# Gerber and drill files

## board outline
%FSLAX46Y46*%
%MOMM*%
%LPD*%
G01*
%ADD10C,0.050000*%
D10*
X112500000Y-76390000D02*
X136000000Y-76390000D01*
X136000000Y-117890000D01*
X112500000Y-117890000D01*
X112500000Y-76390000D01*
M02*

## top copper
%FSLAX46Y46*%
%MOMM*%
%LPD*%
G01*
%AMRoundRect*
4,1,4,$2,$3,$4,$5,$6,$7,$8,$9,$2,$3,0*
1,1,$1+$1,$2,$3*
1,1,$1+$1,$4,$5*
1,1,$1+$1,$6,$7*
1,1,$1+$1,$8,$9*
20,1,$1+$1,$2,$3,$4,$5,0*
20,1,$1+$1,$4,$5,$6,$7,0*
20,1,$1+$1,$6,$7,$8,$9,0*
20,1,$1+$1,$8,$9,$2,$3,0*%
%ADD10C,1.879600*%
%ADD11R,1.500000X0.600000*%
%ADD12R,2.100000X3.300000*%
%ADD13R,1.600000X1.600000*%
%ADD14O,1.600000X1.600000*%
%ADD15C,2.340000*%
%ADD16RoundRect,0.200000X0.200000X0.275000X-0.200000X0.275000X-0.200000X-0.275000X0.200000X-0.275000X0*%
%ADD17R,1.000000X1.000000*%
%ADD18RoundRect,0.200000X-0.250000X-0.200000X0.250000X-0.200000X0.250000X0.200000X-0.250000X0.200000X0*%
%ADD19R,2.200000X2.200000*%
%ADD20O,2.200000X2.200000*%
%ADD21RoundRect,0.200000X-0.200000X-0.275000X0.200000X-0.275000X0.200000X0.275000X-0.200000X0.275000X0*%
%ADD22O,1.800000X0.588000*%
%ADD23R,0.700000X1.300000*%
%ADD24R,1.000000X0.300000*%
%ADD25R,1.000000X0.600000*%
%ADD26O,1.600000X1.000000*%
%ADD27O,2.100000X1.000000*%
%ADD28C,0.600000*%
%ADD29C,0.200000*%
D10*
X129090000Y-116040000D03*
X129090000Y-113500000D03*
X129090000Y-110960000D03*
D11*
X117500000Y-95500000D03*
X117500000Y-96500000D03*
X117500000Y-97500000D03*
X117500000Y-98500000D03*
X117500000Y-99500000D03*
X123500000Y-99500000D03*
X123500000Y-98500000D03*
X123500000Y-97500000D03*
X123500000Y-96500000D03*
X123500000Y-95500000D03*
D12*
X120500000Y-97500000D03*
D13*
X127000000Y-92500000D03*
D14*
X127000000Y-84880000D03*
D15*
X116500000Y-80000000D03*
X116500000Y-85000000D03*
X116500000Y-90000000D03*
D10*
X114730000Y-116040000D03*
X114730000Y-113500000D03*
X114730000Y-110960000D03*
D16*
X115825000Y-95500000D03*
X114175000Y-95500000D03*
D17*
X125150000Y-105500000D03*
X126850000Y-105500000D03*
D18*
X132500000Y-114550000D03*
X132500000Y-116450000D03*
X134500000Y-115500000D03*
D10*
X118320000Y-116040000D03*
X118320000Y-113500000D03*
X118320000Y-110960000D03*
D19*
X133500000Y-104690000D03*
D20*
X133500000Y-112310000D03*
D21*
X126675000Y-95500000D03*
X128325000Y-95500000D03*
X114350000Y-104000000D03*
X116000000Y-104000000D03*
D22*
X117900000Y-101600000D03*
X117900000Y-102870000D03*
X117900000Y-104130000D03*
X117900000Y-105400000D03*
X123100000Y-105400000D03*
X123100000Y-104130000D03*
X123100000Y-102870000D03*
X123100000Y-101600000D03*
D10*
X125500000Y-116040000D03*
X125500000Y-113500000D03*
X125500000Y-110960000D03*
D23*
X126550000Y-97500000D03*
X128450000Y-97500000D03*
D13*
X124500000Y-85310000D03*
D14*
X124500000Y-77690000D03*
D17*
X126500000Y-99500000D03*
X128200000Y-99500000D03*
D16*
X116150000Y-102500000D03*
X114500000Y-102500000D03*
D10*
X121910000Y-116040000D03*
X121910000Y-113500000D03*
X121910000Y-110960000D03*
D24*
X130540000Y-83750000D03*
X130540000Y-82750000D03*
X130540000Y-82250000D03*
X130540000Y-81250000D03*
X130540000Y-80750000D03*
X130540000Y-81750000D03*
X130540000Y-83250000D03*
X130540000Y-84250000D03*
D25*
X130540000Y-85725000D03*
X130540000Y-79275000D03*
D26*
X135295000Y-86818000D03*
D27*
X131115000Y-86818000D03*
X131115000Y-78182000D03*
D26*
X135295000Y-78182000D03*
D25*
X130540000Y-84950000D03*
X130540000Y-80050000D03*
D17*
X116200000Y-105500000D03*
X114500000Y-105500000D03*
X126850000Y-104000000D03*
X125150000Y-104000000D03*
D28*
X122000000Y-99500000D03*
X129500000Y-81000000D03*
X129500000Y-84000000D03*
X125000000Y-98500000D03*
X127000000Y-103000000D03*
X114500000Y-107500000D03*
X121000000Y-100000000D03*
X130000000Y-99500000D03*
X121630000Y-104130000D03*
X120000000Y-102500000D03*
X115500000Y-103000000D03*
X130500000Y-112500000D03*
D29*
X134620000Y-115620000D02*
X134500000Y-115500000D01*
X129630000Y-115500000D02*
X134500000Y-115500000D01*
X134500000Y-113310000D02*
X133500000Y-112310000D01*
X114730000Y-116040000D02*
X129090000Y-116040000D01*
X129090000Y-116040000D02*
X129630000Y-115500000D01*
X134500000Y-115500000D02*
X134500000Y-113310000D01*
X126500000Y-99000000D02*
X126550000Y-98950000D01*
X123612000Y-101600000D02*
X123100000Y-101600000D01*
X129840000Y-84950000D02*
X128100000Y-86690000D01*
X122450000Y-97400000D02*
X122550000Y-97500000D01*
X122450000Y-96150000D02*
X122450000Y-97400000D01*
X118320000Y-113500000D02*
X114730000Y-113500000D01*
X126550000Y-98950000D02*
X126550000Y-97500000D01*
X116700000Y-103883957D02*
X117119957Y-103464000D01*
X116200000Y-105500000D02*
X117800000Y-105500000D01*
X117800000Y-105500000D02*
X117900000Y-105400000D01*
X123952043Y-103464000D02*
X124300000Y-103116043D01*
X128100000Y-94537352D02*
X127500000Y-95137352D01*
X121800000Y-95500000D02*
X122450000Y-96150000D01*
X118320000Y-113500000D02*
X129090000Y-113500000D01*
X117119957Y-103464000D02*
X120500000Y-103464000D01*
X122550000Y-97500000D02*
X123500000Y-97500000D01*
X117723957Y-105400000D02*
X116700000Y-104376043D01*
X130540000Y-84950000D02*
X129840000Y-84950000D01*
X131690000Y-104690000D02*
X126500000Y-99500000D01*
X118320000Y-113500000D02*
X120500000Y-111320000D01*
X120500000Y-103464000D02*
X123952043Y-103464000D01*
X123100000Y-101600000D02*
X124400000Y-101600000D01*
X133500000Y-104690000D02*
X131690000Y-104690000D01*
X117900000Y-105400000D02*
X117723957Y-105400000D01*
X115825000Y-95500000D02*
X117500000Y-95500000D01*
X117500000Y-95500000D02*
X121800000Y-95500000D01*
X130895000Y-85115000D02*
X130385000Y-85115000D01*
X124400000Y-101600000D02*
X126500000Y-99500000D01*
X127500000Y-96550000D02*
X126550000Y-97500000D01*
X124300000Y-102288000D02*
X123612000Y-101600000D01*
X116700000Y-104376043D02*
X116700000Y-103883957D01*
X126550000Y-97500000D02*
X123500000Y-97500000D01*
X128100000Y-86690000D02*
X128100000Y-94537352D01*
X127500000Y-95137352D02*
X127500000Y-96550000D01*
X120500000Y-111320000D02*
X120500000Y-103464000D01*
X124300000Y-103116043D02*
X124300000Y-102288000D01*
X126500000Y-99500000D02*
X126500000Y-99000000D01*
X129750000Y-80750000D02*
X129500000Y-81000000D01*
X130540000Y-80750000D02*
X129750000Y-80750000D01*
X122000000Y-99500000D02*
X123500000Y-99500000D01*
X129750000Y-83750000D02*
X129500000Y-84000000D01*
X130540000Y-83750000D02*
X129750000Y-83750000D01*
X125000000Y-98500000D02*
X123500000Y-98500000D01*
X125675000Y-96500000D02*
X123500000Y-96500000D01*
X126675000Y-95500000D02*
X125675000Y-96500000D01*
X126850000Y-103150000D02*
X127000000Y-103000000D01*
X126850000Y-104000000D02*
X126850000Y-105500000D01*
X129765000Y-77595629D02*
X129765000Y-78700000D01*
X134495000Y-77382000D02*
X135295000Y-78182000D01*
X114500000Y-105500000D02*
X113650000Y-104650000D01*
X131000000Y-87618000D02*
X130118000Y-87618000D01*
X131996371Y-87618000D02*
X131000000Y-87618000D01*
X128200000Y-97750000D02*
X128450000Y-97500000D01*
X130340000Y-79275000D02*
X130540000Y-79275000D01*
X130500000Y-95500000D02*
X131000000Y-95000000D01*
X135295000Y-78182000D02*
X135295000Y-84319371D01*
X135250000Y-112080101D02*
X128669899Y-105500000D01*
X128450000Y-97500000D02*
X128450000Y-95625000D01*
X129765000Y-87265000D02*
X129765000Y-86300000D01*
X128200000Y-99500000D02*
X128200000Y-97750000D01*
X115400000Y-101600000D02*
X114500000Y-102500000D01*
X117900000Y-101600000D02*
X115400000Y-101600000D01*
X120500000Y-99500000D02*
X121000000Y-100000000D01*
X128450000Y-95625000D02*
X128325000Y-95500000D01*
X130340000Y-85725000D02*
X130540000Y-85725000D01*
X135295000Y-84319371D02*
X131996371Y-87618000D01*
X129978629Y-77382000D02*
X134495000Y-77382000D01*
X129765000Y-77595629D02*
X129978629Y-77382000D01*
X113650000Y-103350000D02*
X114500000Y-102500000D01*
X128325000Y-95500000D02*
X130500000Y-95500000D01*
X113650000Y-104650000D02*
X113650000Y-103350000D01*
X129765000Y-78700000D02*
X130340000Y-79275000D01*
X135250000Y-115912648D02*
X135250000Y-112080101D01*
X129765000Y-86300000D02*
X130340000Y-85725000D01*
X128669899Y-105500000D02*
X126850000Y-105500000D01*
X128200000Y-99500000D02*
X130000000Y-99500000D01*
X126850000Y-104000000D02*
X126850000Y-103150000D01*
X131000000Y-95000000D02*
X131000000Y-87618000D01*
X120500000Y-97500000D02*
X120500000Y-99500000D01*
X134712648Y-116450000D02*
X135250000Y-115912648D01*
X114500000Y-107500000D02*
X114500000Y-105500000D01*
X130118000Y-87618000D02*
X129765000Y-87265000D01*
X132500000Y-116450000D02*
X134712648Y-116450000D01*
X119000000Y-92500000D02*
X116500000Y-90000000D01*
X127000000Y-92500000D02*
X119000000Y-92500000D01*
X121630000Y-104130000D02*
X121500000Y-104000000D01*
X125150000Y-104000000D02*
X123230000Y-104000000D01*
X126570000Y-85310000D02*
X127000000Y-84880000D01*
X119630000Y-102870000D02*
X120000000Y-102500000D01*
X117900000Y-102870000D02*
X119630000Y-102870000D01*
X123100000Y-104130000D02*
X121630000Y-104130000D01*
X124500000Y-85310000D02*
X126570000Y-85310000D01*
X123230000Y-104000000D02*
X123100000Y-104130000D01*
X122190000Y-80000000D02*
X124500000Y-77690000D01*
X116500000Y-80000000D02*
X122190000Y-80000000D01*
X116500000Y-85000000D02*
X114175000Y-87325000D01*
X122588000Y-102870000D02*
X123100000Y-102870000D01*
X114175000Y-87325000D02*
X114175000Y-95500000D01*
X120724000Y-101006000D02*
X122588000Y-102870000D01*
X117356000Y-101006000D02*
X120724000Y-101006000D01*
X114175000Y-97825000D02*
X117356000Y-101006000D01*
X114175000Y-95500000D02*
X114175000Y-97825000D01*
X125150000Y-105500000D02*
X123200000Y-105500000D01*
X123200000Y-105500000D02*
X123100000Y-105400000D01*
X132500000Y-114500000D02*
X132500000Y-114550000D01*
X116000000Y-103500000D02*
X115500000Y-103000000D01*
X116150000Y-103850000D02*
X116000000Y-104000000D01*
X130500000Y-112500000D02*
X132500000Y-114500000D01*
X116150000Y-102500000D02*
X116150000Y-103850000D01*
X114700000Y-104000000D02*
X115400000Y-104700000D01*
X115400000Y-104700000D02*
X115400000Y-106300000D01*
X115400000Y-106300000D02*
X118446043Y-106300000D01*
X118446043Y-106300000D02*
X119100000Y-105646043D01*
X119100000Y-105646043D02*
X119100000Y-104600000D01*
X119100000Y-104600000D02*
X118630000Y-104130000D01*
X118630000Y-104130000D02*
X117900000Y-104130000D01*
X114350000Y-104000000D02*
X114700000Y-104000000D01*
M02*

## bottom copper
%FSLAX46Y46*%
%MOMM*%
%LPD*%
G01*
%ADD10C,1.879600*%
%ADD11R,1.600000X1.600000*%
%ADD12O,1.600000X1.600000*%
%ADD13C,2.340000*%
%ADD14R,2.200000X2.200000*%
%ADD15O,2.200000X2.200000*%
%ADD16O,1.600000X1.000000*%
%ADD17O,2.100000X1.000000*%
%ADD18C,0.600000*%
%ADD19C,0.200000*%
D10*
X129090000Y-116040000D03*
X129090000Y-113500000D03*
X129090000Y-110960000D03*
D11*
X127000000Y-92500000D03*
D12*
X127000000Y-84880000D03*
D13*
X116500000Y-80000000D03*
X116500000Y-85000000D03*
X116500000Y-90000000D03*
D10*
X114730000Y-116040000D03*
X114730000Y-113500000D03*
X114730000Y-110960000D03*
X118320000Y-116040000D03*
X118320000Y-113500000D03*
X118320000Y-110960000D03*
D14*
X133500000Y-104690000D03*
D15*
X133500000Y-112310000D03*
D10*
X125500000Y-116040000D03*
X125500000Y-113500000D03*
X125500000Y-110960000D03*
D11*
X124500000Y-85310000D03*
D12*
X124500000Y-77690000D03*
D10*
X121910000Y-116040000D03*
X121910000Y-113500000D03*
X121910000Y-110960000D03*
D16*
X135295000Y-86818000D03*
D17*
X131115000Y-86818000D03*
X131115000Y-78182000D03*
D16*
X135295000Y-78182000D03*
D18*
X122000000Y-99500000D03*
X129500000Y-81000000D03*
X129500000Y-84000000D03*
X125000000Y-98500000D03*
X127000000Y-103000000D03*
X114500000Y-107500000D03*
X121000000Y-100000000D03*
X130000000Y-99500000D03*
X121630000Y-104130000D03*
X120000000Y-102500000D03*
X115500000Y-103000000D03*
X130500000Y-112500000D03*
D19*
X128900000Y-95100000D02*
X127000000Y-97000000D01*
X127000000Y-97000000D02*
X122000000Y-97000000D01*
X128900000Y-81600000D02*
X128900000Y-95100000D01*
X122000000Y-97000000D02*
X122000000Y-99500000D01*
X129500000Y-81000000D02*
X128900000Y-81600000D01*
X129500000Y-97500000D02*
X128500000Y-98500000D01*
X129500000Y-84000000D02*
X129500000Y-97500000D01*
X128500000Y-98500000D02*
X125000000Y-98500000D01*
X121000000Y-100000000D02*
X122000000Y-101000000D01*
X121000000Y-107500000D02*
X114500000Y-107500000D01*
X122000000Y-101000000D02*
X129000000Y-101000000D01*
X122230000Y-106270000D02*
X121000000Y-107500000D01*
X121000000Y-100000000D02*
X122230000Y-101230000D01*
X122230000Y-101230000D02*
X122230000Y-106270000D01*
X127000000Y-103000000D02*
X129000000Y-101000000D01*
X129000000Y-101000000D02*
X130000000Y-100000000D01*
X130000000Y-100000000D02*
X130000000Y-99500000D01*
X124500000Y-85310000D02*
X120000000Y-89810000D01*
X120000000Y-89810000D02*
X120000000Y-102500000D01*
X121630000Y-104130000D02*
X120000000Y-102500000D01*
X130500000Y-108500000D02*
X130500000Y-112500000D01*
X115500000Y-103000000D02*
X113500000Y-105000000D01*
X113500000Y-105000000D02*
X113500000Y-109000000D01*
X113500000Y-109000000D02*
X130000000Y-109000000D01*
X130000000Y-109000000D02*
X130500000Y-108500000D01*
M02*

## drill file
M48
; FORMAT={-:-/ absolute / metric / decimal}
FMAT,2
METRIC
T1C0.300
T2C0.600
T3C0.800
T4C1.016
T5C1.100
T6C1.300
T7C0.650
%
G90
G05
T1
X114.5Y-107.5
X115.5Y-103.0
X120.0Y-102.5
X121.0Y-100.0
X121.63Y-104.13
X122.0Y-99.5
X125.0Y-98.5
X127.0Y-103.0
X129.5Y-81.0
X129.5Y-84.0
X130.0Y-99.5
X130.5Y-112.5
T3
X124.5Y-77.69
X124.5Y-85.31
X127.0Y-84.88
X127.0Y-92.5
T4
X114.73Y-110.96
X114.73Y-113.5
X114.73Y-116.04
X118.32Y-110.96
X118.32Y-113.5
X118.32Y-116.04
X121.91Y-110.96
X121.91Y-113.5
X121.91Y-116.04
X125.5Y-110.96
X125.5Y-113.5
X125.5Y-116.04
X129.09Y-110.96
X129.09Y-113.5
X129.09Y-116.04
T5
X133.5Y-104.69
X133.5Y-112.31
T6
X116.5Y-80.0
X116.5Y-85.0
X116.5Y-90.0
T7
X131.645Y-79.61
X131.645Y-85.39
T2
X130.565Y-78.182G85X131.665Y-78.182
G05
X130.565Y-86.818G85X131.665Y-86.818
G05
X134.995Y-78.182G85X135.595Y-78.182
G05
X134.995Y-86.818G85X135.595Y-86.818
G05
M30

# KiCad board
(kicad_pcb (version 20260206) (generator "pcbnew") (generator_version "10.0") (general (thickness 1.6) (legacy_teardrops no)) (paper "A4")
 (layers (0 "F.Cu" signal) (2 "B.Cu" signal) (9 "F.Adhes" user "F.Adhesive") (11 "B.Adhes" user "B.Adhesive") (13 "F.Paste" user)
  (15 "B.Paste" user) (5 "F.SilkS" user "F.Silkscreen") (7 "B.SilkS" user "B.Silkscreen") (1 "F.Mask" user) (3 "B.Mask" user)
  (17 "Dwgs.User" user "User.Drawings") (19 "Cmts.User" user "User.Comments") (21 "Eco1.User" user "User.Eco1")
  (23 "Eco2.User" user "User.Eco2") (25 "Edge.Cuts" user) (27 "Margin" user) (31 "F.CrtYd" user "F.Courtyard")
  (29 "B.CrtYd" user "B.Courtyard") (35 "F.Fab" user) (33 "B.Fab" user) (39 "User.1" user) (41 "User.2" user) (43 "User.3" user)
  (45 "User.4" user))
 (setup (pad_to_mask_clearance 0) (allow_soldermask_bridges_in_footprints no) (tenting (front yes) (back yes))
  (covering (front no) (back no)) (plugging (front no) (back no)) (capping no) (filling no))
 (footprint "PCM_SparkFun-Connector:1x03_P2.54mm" (layer "F.Cu") (at 129.09 116.04 90)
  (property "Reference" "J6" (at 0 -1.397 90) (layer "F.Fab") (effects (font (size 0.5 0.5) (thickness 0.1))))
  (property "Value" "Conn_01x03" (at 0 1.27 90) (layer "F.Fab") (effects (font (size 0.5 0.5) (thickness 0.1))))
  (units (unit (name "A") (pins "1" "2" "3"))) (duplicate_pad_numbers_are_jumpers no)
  (pad "1" thru_hole circle (at 0 0 180) (size 1.8796 1.8796) (drill 1.016) (layers "*.Cu" "*.Mask") (remove_unused_layers yes)
   (keep_end_layers yes) (zone_layer_connections) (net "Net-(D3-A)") (thermal_bridge_angle 0))
  (pad "2" thru_hole circle (at 2.54 0 180) (size 1.8796 1.8796) (drill 1.016) (layers "*.Cu" "*.Mask") (remove_unused_layers yes)
   (keep_end_layers yes) (zone_layer_connections) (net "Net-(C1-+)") (thermal_bridge_angle 0))
  (pad "3" thru_hole circle (at 5.08 0 180) (size 1.8796 1.8796) (drill 1.016) (layers "*.Cu" "*.Mask") (remove_unused_layers yes)
   (keep_end_layers yes) (zone_layer_connections) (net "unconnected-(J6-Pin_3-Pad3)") (thermal_bridge_angle 0)))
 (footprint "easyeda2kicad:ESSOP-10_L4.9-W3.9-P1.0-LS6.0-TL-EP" (layer "F.Cu") (at 120.5 97.5 -90)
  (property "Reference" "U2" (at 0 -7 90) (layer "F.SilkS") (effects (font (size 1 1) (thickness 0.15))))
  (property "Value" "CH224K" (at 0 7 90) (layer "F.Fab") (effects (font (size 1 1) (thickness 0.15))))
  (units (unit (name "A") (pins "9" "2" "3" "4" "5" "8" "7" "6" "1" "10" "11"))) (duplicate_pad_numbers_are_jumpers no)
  (pad "1" smd rect (at -2 3) (size 1.5 0.6) (layers "F.Cu" "F.Mask" "F.Paste") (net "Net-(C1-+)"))
  (pad "2" smd rect (at -1 3) (size 1.5 0.6) (layers "F.Cu" "F.Mask" "F.Paste") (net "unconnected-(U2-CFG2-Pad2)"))
  (pad "3" smd rect (at 0 3) (size 1.5 0.6) (layers "F.Cu" "F.Mask" "F.Paste") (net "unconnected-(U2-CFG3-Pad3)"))
  (pad "4" smd rect (at 1 3) (size 1.5 0.6) (layers "F.Cu" "F.Mask" "F.Paste") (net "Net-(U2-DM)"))
  (pad "5" smd rect (at 2 3) (size 1.5 0.6) (layers "F.Cu" "F.Mask" "F.Paste") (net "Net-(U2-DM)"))
  (pad "6" smd rect (at 2 -3) (size 1.5 0.6) (layers "F.Cu" "F.Mask" "F.Paste") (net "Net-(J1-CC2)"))
  (pad "7" smd rect (at 1 -3) (size 1.5 0.6) (layers "F.Cu" "F.Mask" "F.Paste") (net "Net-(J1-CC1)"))
  (pad "8" smd rect (at 0 -3) (size 1.5 0.6) (layers "F.Cu" "F.Mask" "F.Paste") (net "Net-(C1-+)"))
  (pad "9" smd rect (at -1 -3) (size 1.5 0.6) (layers "F.Cu" "F.Mask" "F.Paste") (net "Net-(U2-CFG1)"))
  (pad "10" smd rect (at -2 -3) (size 1.5 0.6) (layers "F.Cu" "F.Mask" "F.Paste") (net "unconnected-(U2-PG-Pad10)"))
  (pad "11" smd rect (at 0 0 90) (size 3.3 2.1) (layers "F.Cu" "F.Mask" "F.Paste") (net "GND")))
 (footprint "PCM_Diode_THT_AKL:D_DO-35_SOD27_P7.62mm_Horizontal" (layer "F.Cu") (at 127 92.5 90)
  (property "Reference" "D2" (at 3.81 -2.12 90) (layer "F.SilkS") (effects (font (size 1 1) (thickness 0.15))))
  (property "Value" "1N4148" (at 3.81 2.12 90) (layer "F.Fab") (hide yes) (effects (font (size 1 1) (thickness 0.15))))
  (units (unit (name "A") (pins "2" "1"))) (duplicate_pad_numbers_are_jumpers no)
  (pad "1" thru_hole rect (at 0 0 90) (size 1.6 1.6) (drill 0.8) (layers "*.Cu" "*.Mask") (remove_unused_layers no) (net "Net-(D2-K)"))
  (pad "2" thru_hole oval (at 7.62 0 90) (size 1.6 1.6) (drill 0.8) (layers "*.Cu" "*.Mask") (remove_unused_layers no) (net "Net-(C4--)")))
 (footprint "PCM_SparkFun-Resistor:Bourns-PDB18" (layer "F.Cu") (at 116.5 85 180)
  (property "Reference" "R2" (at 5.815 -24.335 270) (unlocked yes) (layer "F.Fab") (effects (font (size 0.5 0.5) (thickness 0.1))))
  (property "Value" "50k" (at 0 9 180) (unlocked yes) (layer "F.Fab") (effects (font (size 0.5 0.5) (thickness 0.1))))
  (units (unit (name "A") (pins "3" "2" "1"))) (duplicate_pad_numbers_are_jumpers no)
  (pad "1" thru_hole circle (at 0 5 180) (size 2.34 2.34) (drill 1.3) (layers "*.Cu" "*.Mask") (remove_unused_layers no) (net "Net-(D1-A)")
   (thermal_bridge_angle 0))
  (pad "2" thru_hole circle (at 0 0 180) (size 2.34 2.34) (drill 1.3) (layers "*.Cu" "*.Mask") (remove_unused_layers no)
   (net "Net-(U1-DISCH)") (thermal_bridge_angle 0))
  (pad "3" thru_hole circle (at 0 -5 180) (size 2.34 2.34) (drill 1.3) (layers "*.Cu" "*.Mask") (remove_unused_layers no) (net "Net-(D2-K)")
   (thermal_bridge_angle 0)))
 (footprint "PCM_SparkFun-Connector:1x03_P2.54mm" (layer "F.Cu") (at 114.73 116.04 90)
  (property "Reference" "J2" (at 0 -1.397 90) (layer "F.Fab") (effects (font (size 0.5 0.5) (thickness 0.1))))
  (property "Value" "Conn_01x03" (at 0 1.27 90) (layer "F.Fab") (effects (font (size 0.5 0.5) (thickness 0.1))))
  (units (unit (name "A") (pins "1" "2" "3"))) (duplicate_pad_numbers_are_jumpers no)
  (pad "1" thru_hole circle (at 0 0 180) (size 1.8796 1.8796) (drill 1.016) (layers "*.Cu" "*.Mask") (remove_unused_layers yes)
   (keep_end_layers yes) (zone_layer_connections) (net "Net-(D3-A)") (thermal_bridge_angle 0))
  (pad "2" thru_hole circle (at 2.54 0 180) (size 1.8796 1.8796) (drill 1.016) (layers "*.Cu" "*.Mask") (remove_unused_layers yes)
   (keep_end_layers yes) (zone_layer_connections) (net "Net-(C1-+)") (thermal_bridge_angle 0))
  (pad "3" thru_hole circle (at 5.08 0 180) (size 1.8796 1.8796) (drill 1.016) (layers "*.Cu" "*.Mask") (remove_unused_layers yes)
   (keep_end_layers yes) (zone_layer_connections) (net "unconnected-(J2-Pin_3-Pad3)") (thermal_bridge_angle 0)))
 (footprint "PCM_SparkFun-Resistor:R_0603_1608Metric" (layer "F.Cu") (at 115 95.5 180)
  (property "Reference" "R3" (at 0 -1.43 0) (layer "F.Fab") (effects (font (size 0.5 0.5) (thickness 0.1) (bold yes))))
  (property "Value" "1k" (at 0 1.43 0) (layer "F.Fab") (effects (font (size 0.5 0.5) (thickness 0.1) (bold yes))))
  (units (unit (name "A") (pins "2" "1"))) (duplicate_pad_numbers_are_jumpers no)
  (pad "1" smd roundrect (at -0.825 0 180) (size 0.8 0.95) (layers "F.Cu" "F.Mask" "F.Paste") (roundrect_rratio 0.25) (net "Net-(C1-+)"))
  (pad "2" smd roundrect (at 0.825 0 180) (size 0.8 0.95) (layers "F.Cu" "F.Mask" "F.Paste") (roundrect_rratio 0.25) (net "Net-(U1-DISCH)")))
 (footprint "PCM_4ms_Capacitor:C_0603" (layer "F.Cu") (at 126 105.5)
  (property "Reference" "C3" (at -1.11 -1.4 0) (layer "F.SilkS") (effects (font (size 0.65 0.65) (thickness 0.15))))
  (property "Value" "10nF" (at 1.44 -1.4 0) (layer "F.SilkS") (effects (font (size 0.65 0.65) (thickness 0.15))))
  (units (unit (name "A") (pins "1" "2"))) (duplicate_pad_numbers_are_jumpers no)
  (pad "1" smd rect (at -0.85 0) (size 1 1) (layers "F.Cu" "F.Mask" "F.Paste") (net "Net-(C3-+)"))
  (pad "2" smd rect (at 0.85 0) (size 1 1) (layers "F.Cu" "F.Mask" "F.Paste") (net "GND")))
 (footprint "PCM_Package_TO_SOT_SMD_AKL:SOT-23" (layer "F.Cu") (at 133.5 115.5)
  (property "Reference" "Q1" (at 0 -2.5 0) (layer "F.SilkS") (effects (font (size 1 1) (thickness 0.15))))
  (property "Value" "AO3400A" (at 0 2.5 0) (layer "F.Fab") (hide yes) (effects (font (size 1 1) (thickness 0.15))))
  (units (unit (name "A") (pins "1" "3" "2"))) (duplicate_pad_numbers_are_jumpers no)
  (pad "1" smd roundrect (at -1 -0.95) (size 0.9 0.8) (layers "F.Cu" "F.Mask" "F.Paste") (roundrect_rratio 0.25) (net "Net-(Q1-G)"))
  (pad "2" smd roundrect (at -1 0.95) (size 0.9 0.8) (layers "F.Cu" "F.Mask" "F.Paste") (roundrect_rratio 0.25) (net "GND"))
  (pad "3" smd roundrect (at 1 0) (size 0.9 0.8) (layers "F.Cu" "F.Mask" "F.Paste") (roundrect_rratio 0.25) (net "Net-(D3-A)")))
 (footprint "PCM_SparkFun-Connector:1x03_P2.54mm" (layer "F.Cu") (at 118.32 116.04 90)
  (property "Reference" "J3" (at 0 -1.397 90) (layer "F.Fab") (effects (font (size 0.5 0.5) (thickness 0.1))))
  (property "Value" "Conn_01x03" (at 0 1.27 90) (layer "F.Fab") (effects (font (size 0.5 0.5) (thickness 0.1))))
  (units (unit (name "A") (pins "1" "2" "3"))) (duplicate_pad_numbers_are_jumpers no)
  (pad "1" thru_hole circle (at 0 0 180) (size 1.8796 1.8796) (drill 1.016) (layers "*.Cu" "*.Mask") (remove_unused_layers yes)
   (keep_end_layers yes) (zone_layer_connections) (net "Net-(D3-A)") (thermal_bridge_angle 0))
  (pad "2" thru_hole circle (at 2.54 0 180) (size 1.8796 1.8796) (drill 1.016) (layers "*.Cu" "*.Mask") (remove_unused_layers yes)
   (keep_end_layers yes) (zone_layer_connections) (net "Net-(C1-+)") (thermal_bridge_angle 0))
  (pad "3" thru_hole circle (at 5.08 0 180) (size 1.8796 1.8796) (drill 1.016) (layers "*.Cu" "*.Mask") (remove_unused_layers yes)
   (keep_end_layers yes) (zone_layer_connections) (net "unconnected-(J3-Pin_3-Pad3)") (thermal_bridge_angle 0)))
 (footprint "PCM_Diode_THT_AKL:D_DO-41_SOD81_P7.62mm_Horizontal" (layer "F.Cu") (at 133.5 104.69 -90)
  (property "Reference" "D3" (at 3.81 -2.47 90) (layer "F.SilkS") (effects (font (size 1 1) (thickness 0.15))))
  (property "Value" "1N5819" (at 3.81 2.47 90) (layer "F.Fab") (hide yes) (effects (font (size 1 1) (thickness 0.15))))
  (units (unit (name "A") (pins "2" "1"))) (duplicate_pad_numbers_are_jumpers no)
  (pad "1" thru_hole rect (at 0 0 270) (size 2.2 2.2) (drill 1.1) (layers "*.Cu" "*.Mask") (remove_unused_layers no) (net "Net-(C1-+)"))
  (pad "2" thru_hole oval (at 7.62 0 270) (size 2.2 2.2) (drill 1.1) (layers "*.Cu" "*.Mask") (remove_unused_layers no) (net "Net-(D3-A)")))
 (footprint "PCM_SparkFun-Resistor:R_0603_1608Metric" (layer "F.Cu") (at 127.5 95.5)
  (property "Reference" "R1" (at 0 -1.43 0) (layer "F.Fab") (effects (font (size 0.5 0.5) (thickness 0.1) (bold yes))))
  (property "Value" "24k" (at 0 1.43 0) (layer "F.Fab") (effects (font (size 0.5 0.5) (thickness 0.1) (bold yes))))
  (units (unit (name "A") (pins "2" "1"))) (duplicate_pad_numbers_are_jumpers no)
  (pad "1" smd roundrect (at -0.825 0) (size 0.8 0.95) (layers "F.Cu" "F.Mask" "F.Paste") (roundrect_rratio 0.25) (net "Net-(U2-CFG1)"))
  (pad "2" smd roundrect (at 0.825 0) (size 0.8 0.95) (layers "F.Cu" "F.Mask" "F.Paste") (roundrect_rratio 0.25) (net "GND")))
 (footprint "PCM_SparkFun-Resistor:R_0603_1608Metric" (layer "F.Cu") (at 115.175 104)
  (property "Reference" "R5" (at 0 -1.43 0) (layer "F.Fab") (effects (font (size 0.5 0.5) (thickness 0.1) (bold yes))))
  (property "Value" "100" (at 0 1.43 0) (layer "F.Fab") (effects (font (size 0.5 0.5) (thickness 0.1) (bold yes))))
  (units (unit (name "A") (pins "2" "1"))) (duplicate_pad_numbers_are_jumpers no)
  (pad "1" smd roundrect (at -0.825 0) (size 0.8 0.95) (layers "F.Cu" "F.Mask" "F.Paste") (roundrect_rratio 0.25) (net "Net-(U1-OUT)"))
  (pad "2" smd roundrect (at 0.825 0) (size 0.8 0.95) (layers "F.Cu" "F.Mask" "F.Paste") (roundrect_rratio 0.25) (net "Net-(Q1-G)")))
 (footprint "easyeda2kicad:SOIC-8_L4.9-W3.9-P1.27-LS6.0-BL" (layer "F.Cu") (at 120.5 103.5 -90)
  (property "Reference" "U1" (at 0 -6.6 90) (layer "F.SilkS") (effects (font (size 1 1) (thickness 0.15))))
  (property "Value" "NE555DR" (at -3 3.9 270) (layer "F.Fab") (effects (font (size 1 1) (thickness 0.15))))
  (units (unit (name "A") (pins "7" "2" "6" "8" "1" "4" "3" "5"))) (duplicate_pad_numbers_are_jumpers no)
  (pad "1" smd oval (at -1.9 2.6 270) (size 0.588 1.8) (layers "F.Cu" "F.Mask" "F.Paste") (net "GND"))
  (pad "2" smd oval (at -0.63 2.6 270) (size 0.588 1.8) (layers "F.Cu" "F.Mask" "F.Paste") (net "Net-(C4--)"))
  (pad "3" smd oval (at 0.63 2.6 270) (size 0.588 1.8) (layers "F.Cu" "F.Mask" "F.Paste") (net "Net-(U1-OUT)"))
  (pad "4" smd oval (at 1.9 2.6 270) (size 0.588 1.8) (layers "F.Cu" "F.Mask" "F.Paste") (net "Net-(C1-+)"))
  (pad "5" smd oval (at 1.9 -2.6 270) (size 0.588 1.8) (layers "F.Cu" "F.Mask" "F.Paste") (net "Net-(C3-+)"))
  (pad "6" smd oval (at 0.63 -2.6 270) (size 0.588 1.8) (layers "F.Cu" "F.Mask" "F.Paste") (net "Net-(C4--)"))
  (pad "7" smd oval (at -0.63 -2.6 270) (size 0.588 1.8) (layers "F.Cu" "F.Mask" "F.Paste") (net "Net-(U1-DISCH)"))
  (pad "8" smd oval (at -1.9 -2.6 270) (size 0.588 1.8) (layers "F.Cu" "F.Mask" "F.Paste") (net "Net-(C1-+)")))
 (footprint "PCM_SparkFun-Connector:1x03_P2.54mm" (layer "F.Cu") (at 125.5 116.04 90)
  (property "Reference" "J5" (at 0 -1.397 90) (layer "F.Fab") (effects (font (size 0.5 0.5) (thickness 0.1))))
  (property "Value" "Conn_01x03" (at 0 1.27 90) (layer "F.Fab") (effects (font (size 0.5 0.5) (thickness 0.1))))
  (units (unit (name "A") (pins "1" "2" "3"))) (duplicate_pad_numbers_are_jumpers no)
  (pad "1" thru_hole circle (at 0 0 180) (size 1.8796 1.8796) (drill 1.016) (layers "*.Cu" "*.Mask") (remove_unused_layers yes)
   (keep_end_layers yes) (zone_layer_connections) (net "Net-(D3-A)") (thermal_bridge_angle 0))
  (pad "2" thru_hole circle (at 2.54 0 180) (size 1.8796 1.8796) (drill 1.016) (layers "*.Cu" "*.Mask") (remove_unused_layers yes)
   (keep_end_layers yes) (zone_layer_connections) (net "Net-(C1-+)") (thermal_bridge_angle 0))
  (pad "3" thru_hole circle (at 5.08 0 180) (size 1.8796 1.8796) (drill 1.016) (layers "*.Cu" "*.Mask") (remove_unused_layers yes)
   (keep_end_layers yes) (zone_layer_connections) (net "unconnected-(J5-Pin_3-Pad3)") (thermal_bridge_angle 0)))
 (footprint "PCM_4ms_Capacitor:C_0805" (layer "F.Cu") (at 127.5 97.5)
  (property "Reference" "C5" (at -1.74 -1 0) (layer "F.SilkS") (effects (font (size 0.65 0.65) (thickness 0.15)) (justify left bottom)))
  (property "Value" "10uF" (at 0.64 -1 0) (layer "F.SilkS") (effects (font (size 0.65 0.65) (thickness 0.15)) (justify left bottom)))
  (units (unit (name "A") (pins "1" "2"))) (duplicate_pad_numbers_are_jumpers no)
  (pad "1" smd rect (at -0.95 0) (size 0.7 1.3) (layers "F.Cu" "F.Mask" "F.Paste") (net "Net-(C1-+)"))
  (pad "2" smd rect (at 0.95 0) (size 0.7 1.3) (layers "F.Cu" "F.Mask" "F.Paste") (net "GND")))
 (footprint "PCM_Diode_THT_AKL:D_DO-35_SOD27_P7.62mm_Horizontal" (layer "F.Cu") (at 124.5 85.31 90)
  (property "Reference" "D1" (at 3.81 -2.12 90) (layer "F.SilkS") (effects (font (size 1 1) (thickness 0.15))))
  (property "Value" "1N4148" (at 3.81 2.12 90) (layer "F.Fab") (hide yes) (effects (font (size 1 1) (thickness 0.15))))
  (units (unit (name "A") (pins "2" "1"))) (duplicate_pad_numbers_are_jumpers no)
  (pad "1" thru_hole rect (at 0 0 90) (size 1.6 1.6) (drill 0.8) (layers "*.Cu" "*.Mask") (remove_unused_layers no) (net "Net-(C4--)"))
  (pad "2" thru_hole oval (at 7.62 0 90) (size 1.6 1.6) (drill 0.8) (layers "*.Cu" "*.Mask") (remove_unused_layers no) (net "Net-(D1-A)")))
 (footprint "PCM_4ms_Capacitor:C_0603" (layer "F.Cu") (at 127.35 99.5)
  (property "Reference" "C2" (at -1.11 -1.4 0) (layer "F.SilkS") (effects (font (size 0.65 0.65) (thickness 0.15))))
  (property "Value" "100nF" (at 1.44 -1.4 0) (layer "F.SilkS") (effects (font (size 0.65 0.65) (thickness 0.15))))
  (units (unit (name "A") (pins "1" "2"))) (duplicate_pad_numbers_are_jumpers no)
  (pad "1" smd rect (at -0.85 0) (size 1 1) (layers "F.Cu" "F.Mask" "F.Paste") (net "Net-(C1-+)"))
  (pad "2" smd rect (at 0.85 0) (size 1 1) (layers "F.Cu" "F.Mask" "F.Paste") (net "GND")))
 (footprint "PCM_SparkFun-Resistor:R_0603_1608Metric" (layer "F.Cu") (at 115.325 102.5 180)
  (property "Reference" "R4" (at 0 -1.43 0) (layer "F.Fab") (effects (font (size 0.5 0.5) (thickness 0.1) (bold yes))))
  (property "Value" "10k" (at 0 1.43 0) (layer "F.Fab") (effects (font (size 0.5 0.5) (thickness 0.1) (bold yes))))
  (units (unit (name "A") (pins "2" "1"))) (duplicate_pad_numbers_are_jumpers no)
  (pad "1" smd roundrect (at -0.825 0 180) (size 0.8 0.95) (layers "F.Cu" "F.Mask" "F.Paste") (roundrect_rratio 0.25) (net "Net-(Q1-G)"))
  (pad "2" smd roundrect (at 0.825 0 180) (size 0.8 0.95) (layers "F.Cu" "F.Mask" "F.Paste") (roundrect_rratio 0.25) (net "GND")))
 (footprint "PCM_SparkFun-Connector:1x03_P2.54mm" (layer "F.Cu") (at 121.91 116.04 90)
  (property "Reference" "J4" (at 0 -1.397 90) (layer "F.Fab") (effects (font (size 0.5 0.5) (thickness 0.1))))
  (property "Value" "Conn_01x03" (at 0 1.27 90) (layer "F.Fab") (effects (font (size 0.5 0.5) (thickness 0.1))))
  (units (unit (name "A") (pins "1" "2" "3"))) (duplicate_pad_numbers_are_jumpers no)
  (pad "1" thru_hole circle (at 0 0 180) (size 1.8796 1.8796) (drill 1.016) (layers "*.Cu" "*.Mask") (remove_unused_layers yes)
   (keep_end_layers yes) (zone_layer_connections) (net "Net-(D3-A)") (thermal_bridge_angle 0))
  (pad "2" thru_hole circle (at 2.54 0 180) (size 1.8796 1.8796) (drill 1.016) (layers "*.Cu" "*.Mask") (remove_unused_layers yes)
   (keep_end_layers yes) (zone_layer_connections) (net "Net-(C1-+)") (thermal_bridge_angle 0))
  (pad "3" thru_hole circle (at 5.08 0 180) (size 1.8796 1.8796) (drill 1.016) (layers "*.Cu" "*.Mask") (remove_unused_layers yes)
   (keep_end_layers yes) (zone_layer_connections) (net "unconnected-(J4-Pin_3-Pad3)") (thermal_bridge_angle 0)))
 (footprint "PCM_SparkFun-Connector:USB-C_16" (layer "F.Cu") (at 130.2 82.5 90)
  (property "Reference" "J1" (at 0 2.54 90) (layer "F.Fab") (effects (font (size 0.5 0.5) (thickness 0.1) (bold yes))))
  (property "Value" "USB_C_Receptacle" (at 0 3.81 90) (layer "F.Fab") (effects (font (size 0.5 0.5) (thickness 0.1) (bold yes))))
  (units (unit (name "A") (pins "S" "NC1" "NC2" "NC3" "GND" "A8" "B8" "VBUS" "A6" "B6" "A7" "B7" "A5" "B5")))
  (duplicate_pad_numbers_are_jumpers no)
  (pad "" np_thru_hole circle (at -2.89 1.445 90) (size 0.65 0.65) (drill 0.65) (layers "*.Cu" "*.Mask"))
  (pad "" np_thru_hole circle (at 2.89 1.445 90) (size 0.65 0.65) (drill 0.65) (layers "*.Cu" "*.Mask"))
  (pad "A5" smd rect (at -1.25 0.34 270) (size 0.3 1) (layers "F.Cu" "F.Mask" "F.Paste") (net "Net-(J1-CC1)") (thermal_bridge_angle 0))
  (pad "A6" smd rect (at -0.25 0.34 270) (size 0.3 1) (layers "F.Cu" "F.Mask" "F.Paste") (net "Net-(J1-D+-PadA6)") (thermal_bridge_angle 0))
  (pad "A7" smd rect (at 0.25 0.34 90) (size 0.3 1) (layers "F.Cu" "F.Mask" "F.Paste") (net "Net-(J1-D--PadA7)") (thermal_bridge_angle 0))
  (pad "A8" smd rect (at 1.25 0.34 90) (size 0.3 1) (layers "F.Cu" "F.Mask" "F.Paste") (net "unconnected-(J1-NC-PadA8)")
   (thermal_bridge_angle 0))
  (pad "B5" smd rect (at 1.75 0.34 90) (size 0.3 1) (layers "F.Cu" "F.Mask" "F.Paste") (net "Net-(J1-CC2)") (thermal_bridge_angle 0))
  (pad "B6" smd rect (at 0.75 0.34 90) (size 0.3 1) (layers "F.Cu" "F.Mask" "F.Paste") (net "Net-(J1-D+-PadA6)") (thermal_bridge_angle 0))
  (pad "B7" smd rect (at -0.75 0.34 270) (size 0.3 1) (layers "F.Cu" "F.Mask" "F.Paste") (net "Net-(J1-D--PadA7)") (thermal_bridge_angle 0))
  (pad "B8" smd rect (at -1.75 0.34 270) (size 0.3 1) (layers "F.Cu" "F.Mask" "F.Paste") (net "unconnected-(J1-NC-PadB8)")
   (thermal_bridge_angle 0))
  (pad "GND" smd rect (at -3.225 0.34 270) (size 0.6 1) (layers "F.Cu" "F.Mask") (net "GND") (thermal_bridge_angle 0))
  (pad "GND" smd rect (at 3.225 0.34 90) (size 0.6 1) (layers "F.Cu" "F.Mask") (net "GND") (thermal_bridge_angle 0))
  (pad "NC1" thru_hole oval (at -4.318 5.095 90) (size 1 1.6) (drill oval 0.6 1.2) (layers "*.Cu" "*.Mask" "F.Paste")
   (remove_unused_layers no) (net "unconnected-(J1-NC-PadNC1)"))
  (pad "NC2" thru_hole oval (at -4.318 0.915 90) (size 1 2.1) (drill oval 0.6 1.7) (layers "*.Cu" "*.Mask" "F.Paste")
   (remove_unused_layers no) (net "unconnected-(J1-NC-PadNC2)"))
  (pad "NC3" thru_hole oval (at 4.318 0.915 90) (size 1 2.1) (drill oval 0.6 1.7) (layers "*.Cu" "*.Mask" "F.Paste")
   (remove_unused_layers no) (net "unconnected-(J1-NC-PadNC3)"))
  (pad "S" thru_hole oval (at 4.318 5.095 90) (size 1 1.6) (drill oval 0.6 1.2) (layers "*.Cu" "*.Mask" "F.Paste") (remove_unused_layers no)
   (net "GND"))
  (pad "VBUS" smd rect (at -2.45 0.34 270) (size 0.6 1) (layers "F.Cu" "F.Mask") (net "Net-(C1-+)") (thermal_bridge_angle 0))
  (pad "VBUS" smd rect (at 2.45 0.34 90) (size 0.6 1) (layers "F.Cu" "F.Mask") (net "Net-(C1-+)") (thermal_bridge_angle 0)))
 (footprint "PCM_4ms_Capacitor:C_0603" (layer "F.Cu") (at 115.35 105.5 180)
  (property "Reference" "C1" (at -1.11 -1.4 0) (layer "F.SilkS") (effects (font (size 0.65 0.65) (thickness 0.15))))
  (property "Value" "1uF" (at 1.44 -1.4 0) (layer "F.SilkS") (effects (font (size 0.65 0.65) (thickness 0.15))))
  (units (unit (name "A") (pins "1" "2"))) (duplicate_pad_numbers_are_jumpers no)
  (pad "1" smd rect (at -0.85 0 180) (size 1 1) (layers "F.Cu" "F.Mask" "F.Paste") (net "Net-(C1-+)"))
  (pad "2" smd rect (at 0.85 0 180) (size 1 1) (layers "F.Cu" "F.Mask" "F.Paste") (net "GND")))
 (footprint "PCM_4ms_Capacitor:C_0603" (layer "F.Cu") (at 126 104 180)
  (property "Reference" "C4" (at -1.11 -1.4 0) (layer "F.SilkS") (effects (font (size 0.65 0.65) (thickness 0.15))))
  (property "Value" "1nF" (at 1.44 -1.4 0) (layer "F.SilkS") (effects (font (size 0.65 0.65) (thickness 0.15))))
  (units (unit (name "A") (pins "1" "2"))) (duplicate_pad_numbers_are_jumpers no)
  (pad "1" smd rect (at -0.85 0 180) (size 1 1) (layers "F.Cu" "F.Mask" "F.Paste") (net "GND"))
  (pad "2" smd rect (at 0.85 0 180) (size 1 1) (layers "F.Cu" "F.Mask" "F.Paste") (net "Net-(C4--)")))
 (gr_rect (start 112.5 76.39) (end 136 117.89) (stroke (width 0.05) (type default)) (fill no) (layer "Edge.Cuts"))
 (segment (start 134.62 115.62) (end 134.5 115.5) (width 0.2) (layer "F.Cu") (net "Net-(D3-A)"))
 (segment (start 129.63 115.5) (end 134.5 115.5) (width 0.2) (layer "F.Cu") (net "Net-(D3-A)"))
 (segment (start 134.5 113.31) (end 133.5 112.31) (width 0.2) (layer "F.Cu") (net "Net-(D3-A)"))
 (segment (start 114.73 116.04) (end 129.09 116.04) (width 0.2) (layer "F.Cu") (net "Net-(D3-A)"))
 (segment (start 129.09 116.04) (end 129.63 115.5) (width 0.2) (layer "F.Cu") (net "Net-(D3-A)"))
 (segment (start 134.5 115.5) (end 134.5 113.31) (width 0.2) (layer "F.Cu") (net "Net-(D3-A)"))
 (segment (start 126.5 99) (end 126.55 98.95) (width 0.2) (layer "F.Cu") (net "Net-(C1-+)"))
 (segment (start 123.612 101.6) (end 123.1 101.6) (width 0.2) (layer "F.Cu") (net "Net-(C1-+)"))
 (segment (start 129.84 84.95) (end 128.1 86.69) (width 0.2) (layer "F.Cu") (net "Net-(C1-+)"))
 (segment (start 122.45 97.4) (end 122.55 97.5) (width 0.2) (layer "F.Cu") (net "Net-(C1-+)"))
 (segment (start 122.45 96.15) (end 122.45 97.4) (width 0.2) (layer "F.Cu") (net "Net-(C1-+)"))
 (segment (start 118.32 113.5) (end 114.73 113.5) (width 0.2) (layer "F.Cu") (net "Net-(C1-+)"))
 (segment (start 126.55 98.95) (end 126.55 97.5) (width 0.2) (layer "F.Cu") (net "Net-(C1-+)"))
 (segment (start 116.7 103.883957) (end 117.119957 103.464) (width 0.2) (layer "F.Cu") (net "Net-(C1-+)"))
 (segment (start 116.2 105.5) (end 117.8 105.5) (width 0.2) (layer "F.Cu") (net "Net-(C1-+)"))
 (segment (start 117.8 105.5) (end 117.9 105.4) (width 0.2) (layer "F.Cu") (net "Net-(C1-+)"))
 (segment (start 123.952043 103.464) (end 124.3 103.116043) (width 0.2) (layer "F.Cu") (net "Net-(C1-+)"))
 (segment (start 128.1 94.537352) (end 127.5 95.137352) (width 0.2) (layer "F.Cu") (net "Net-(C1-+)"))
 (segment (start 121.8 95.5) (end 122.45 96.15) (width 0.2) (layer "F.Cu") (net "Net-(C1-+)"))
 (segment (start 118.32 113.5) (end 129.09 113.5) (width 0.2) (layer "F.Cu") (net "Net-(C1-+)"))
 (segment (start 117.119957 103.464) (end 120.5 103.464) (width 0.2) (layer "F.Cu") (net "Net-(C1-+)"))
 (segment (start 122.55 97.5) (end 123.5 97.5) (width 0.2) (layer "F.Cu") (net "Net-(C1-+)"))
 (segment (start 117.723957 105.4) (end 116.7 104.376043) (width 0.2) (layer "F.Cu") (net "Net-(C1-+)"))
 (segment (start 130.54 84.95) (end 129.84 84.95) (width 0.2) (layer "F.Cu") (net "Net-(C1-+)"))
 (segment (start 131.69 104.69) (end 126.5 99.5) (width 0.2) (layer "F.Cu") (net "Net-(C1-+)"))
 (segment (start 118.32 113.5) (end 120.5 111.32) (width 0.2) (layer "F.Cu") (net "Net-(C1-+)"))
 (segment (start 120.5 103.464) (end 123.952043 103.464) (width 0.2) (layer "F.Cu") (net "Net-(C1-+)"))
 (segment (start 123.1 101.6) (end 124.4 101.6) (width 0.2) (layer "F.Cu") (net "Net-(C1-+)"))
 (segment (start 133.5 104.69) (end 131.69 104.69) (width 0.2) (layer "F.Cu") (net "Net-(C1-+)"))
 (segment (start 117.9 105.4) (end 117.723957 105.4) (width 0.2) (layer "F.Cu") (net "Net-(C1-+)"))
 (segment (start 115.825 95.5) (end 117.5 95.5) (width 0.2) (layer "F.Cu") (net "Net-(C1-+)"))
 (segment (start 117.5 95.5) (end 121.8 95.5) (width 0.2) (layer "F.Cu") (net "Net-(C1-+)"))
 (segment (start 130.895 85.115) (end 130.385 85.115) (width 0.2) (layer "F.Cu") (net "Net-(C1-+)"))
 (segment (start 124.4 101.6) (end 126.5 99.5) (width 0.2) (layer "F.Cu") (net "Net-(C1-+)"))
 (segment (start 127.5 96.55) (end 126.55 97.5) (width 0.2) (layer "F.Cu") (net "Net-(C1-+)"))
 (segment (start 124.3 102.288) (end 123.612 101.6) (width 0.2) (layer "F.Cu") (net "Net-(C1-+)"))
 (segment (start 116.7 104.376043) (end 116.7 103.883957) (width 0.2) (layer "F.Cu") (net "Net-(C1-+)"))
 (segment (start 126.55 97.5) (end 123.5 97.5) (width 0.2) (layer "F.Cu") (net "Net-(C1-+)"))
 (segment (start 128.1 86.69) (end 128.1 94.537352) (width 0.2) (layer "F.Cu") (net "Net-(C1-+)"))
 (segment (start 127.5 95.137352) (end 127.5 96.55) (width 0.2) (layer "F.Cu") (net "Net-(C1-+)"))
 (segment (start 120.5 111.32) (end 120.5 103.464) (width 0.2) (layer "F.Cu") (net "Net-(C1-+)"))
 (segment (start 124.3 103.116043) (end 124.3 102.288) (width 0.2) (layer "F.Cu") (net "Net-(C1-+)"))
 (segment (start 126.5 99.5) (end 126.5 99) (width 0.2) (layer "F.Cu") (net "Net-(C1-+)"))
 (segment (start 129.75 80.75) (end 129.5 81) (width 0.2) (layer "F.Cu") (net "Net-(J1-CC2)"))
 (segment (start 130.54 80.75) (end 129.75 80.75) (width 0.2) (layer "F.Cu") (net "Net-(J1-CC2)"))
 (segment (start 122 99.5) (end 123.5 99.5) (width 0.2) (layer "F.Cu") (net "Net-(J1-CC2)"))
 (via (at 122 99.5) (size 0.6) (drill 0.3) (layers "F.Cu" "B.Cu") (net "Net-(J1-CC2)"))
 (via (at 129.5 81) (size 0.6) (drill 0.3) (layers "F.Cu" "B.Cu") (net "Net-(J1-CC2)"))
 (segment (start 128.9 95.1) (end 127 97) (width 0.2) (layer "B.Cu") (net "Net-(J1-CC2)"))
 (segment (start 127 97) (end 122 97) (width 0.2) (layer "B.Cu") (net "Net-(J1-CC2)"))
 (segment (start 128.9 81.6) (end 128.9 95.1) (width 0.2) (layer "B.Cu") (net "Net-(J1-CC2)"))
 (segment (start 122 97) (end 122 99.5) (width 0.2) (layer "B.Cu") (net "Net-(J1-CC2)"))
 (segment (start 129.5 81) (end 128.9 81.6) (width 0.2) (layer "B.Cu") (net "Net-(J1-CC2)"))
 (segment (start 129.75 83.75) (end 129.5 84) (width 0.2) (layer "F.Cu") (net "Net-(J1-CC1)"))
 (segment (start 130.54 83.75) (end 129.75 83.75) (width 0.2) (layer "F.Cu") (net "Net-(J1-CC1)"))
 (segment (start 125 98.5) (end 123.5 98.5) (width 0.2) (layer "F.Cu") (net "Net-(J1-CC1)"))
 (via (at 129.5 84) (size 0.6) (drill 0.3) (layers "F.Cu" "B.Cu") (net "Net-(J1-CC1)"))
 (via (at 125 98.5) (size 0.6) (drill 0.3) (layers "F.Cu" "B.Cu") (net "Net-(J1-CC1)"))
 (segment (start 129.5 97.5) (end 128.5 98.5) (width 0.2) (layer "B.Cu") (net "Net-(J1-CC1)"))
 (segment (start 129.5 84) (end 129.5 97.5) (width 0.2) (layer "B.Cu") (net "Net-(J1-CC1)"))
 (segment (start 128.5 98.5) (end 125 98.5) (width 0.2) (layer "B.Cu") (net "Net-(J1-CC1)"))
 (segment (start 125.675 96.5) (end 123.5 96.5) (width 0.2) (layer "F.Cu") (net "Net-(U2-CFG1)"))
 (segment (start 126.675 95.5) (end 125.675 96.5) (width 0.2) (layer "F.Cu") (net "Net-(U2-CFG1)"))
 (segment (start 126.85 103.15) (end 127 103) (width 0.2) (layer "F.Cu") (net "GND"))
 (segment (start 126.85 104) (end 126.85 105.5) (width 0.2) (layer "F.Cu") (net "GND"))
 (segment (start 129.765 77.595629) (end 129.765 78.7) (width 0.2) (layer "F.Cu") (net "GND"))
 (segment (start 134.495 77.382) (end 135.295 78.182) (width 0.2) (layer "F.Cu") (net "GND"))
 (segment (start 114.5 105.5) (end 113.65 104.65) (width 0.2) (layer "F.Cu") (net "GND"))
 (segment (start 131 87.618) (end 130.118 87.618) (width 0.2) (layer "F.Cu") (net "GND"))
 (segment (start 131.996371 87.618) (end 131 87.618) (width 0.2) (layer "F.Cu") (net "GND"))
 (segment (start 128.2 97.75) (end 128.45 97.5) (width 0.2) (layer "F.Cu") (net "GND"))
 (segment (start 130.34 79.275) (end 130.54 79.275) (width 0.2) (layer "F.Cu") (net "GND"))
 (segment (start 130.5 95.5) (end 131 95) (width 0.2) (layer "F.Cu") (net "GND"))
 (segment (start 135.295 78.182) (end 135.295 84.319371) (width 0.2) (layer "F.Cu") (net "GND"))
 (segment (start 135.25 112.080101) (end 128.669899 105.5) (width 0.2) (layer "F.Cu") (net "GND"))
 (segment (start 128.45 97.5) (end 128.45 95.625) (width 0.2) (layer "F.Cu") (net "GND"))
 (segment (start 129.765 87.265) (end 129.765 86.3) (width 0.2) (layer "F.Cu") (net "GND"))
 (segment (start 128.2 99.5) (end 128.2 97.75) (width 0.2) (layer "F.Cu") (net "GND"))
 (segment (start 115.4 101.6) (end 114.5 102.5) (width 0.2) (layer "F.Cu") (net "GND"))
 (segment (start 117.9 101.6) (end 115.4 101.6) (width 0.2) (layer "F.Cu") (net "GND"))
 (segment (start 120.5 99.5) (end 121 100) (width 0.2) (layer "F.Cu") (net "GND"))
 (segment (start 128.45 95.625) (end 128.325 95.5) (width 0.2) (layer "F.Cu") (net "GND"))
 (segment (start 130.34 85.725) (end 130.54 85.725) (width 0.2) (layer "F.Cu") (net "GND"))
 (segment (start 135.295 84.319371) (end 131.996371 87.618) (width 0.2) (layer "F.Cu") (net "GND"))
 (segment (start 129.978629 77.382) (end 134.495 77.382) (width 0.2) (layer "F.Cu") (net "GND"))
 (segment (start 129.765 77.595629) (end 129.978629 77.382) (width 0.2) (layer "F.Cu") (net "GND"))
 (segment (start 113.65 103.35) (end 114.5 102.5) (width 0.2) (layer "F.Cu") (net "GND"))
 (segment (start 128.325 95.5) (end 130.5 95.5) (width 0.2) (layer "F.Cu") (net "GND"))
 (segment (start 113.65 104.65) (end 113.65 103.35) (width 0.2) (layer "F.Cu") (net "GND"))
 (segment (start 129.765 78.7) (end 130.34 79.275) (width 0.2) (layer "F.Cu") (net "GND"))
 (segment (start 135.25 115.912648) (end 135.25 112.080101) (width 0.2) (layer "F.Cu") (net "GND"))
 (segment (start 129.765 86.3) (end 130.34 85.725) (width 0.2) (layer "F.Cu") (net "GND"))
 (segment (start 128.669899 105.5) (end 126.85 105.5) (width 0.2) (layer "F.Cu") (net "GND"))
 (segment (start 128.2 99.5) (end 130 99.5) (width 0.2) (layer "F.Cu") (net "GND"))
 (segment (start 126.85 104) (end 126.85 103.15) (width 0.2) (layer "F.Cu") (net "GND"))
 (segment (start 131 95) (end 131 87.618) (width 0.2) (layer "F.Cu") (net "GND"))
 (segment (start 120.5 97.5) (end 120.5 99.5) (width 0.2) (layer "F.Cu") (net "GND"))
 (segment (start 134.712648 116.45) (end 135.25 115.912648) (width 0.2) (layer "F.Cu") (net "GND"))
 (segment (start 114.5 107.5) (end 114.5 105.5) (width 0.2) (layer "F.Cu") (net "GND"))
 (segment (start 130.118 87.618) (end 129.765 87.265) (width 0.2) (layer "F.Cu") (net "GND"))
 (segment (start 132.5 116.45) (end 134.712648 116.45) (width 0.2) (layer "F.Cu") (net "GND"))
 (via (at 127 103) (size 0.6) (drill 0.3) (layers "F.Cu" "B.Cu") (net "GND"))
 (via (at 114.5 107.5) (size 0.6) (drill 0.3) (layers "F.Cu" "B.Cu") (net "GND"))
 (via (at 121 100) (size 0.6) (drill 0.3) (layers "F.Cu" "B.Cu") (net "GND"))
 (via (at 130 99.5) (size 0.6) (drill 0.3) (layers "F.Cu" "B.Cu") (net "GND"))
 (segment (start 121 100) (end 122 101) (width 0.2) (layer "B.Cu") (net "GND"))
 (segment (start 121 107.5) (end 114.5 107.5) (width 0.2) (layer "B.Cu") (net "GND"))
 (segment (start 122 101) (end 129 101) (width 0.2) (layer "B.Cu") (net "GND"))
 (segment (start 122.23 106.27) (end 121 107.5) (width 0.2) (layer "B.Cu") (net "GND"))
 (segment (start 121 100) (end 122.23 101.23) (width 0.2) (layer "B.Cu") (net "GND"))
 (segment (start 122.23 101.23) (end 122.23 106.27) (width 0.2) (layer "B.Cu") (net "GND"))
 (segment (start 127 103) (end 129 101) (width 0.2) (layer "B.Cu") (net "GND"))
 (segment (start 129 101) (end 130 100) (width 0.2) (layer "B.Cu") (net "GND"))
 (segment (start 130 100) (end 130 99.5) (width 0.2) (layer "B.Cu") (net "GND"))
 (segment (start 119 92.5) (end 116.5 90) (width 0.2) (layer "F.Cu") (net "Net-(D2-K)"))
 (segment (start 127 92.5) (end 119 92.5) (width 0.2) (layer "F.Cu") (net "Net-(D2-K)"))
 (segment (start 121.63 104.13) (end 121.5 104) (width 0.2) (layer "F.Cu") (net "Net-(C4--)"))
 (segment (start 125.15 104) (end 123.23 104) (width 0.2) (layer "F.Cu") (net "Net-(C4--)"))
 (segment (start 126.57 85.31) (end 127 84.88) (width 0.2) (layer "F.Cu") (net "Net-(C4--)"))
 (segment (start 119.63 102.87) (end 120 102.5) (width 0.2) (layer "F.Cu") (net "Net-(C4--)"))
 (segment (start 117.9 102.87) (end 119.63 102.87) (width 0.2) (layer "F.Cu") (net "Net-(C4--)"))
 (segment (start 123.1 104.13) (end 121.63 104.13) (width 0.2) (layer "F.Cu") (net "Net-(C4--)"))
 (segment (start 124.5 85.31) (end 126.57 85.31) (width 0.2) (layer "F.Cu") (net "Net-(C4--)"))
 (segment (start 123.23 104) (end 123.1 104.13) (width 0.2) (layer "F.Cu") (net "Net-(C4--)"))
 (via (at 121.63 104.13) (size 0.6) (drill 0.3) (layers "F.Cu" "B.Cu") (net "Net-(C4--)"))
 (via (at 120 102.5) (size 0.6) (drill 0.3) (layers "F.Cu" "B.Cu") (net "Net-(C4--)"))
 (segment (start 124.5 85.31) (end 120 89.81) (width 0.2) (layer "B.Cu") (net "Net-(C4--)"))
 (segment (start 120 89.81) (end 120 102.5) (width 0.2) (layer "B.Cu") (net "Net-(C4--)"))
 (segment (start 121.63 104.13) (end 120 102.5) (width 0.2) (layer "B.Cu") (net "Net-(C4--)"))
 (segment (start 122.19 80) (end 124.5 77.69) (width 0.2) (layer "F.Cu") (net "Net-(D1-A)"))
 (segment (start 116.5 80) (end 122.19 80) (width 0.2) (layer "F.Cu") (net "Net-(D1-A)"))
 (segment (start 116.5 85) (end 114.175 87.325) (width 0.2) (layer "F.Cu") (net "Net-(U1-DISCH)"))
 (segment (start 122.588 102.87) (end 123.1 102.87) (width 0.2) (layer "F.Cu") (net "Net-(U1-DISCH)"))
 (segment (start 114.175 87.325) (end 114.175 95.5) (width 0.2) (layer "F.Cu") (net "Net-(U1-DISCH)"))
 (segment (start 120.724 101.006) (end 122.588 102.87) (width 0.2) (layer "F.Cu") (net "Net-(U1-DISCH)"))
 (segment (start 117.356 101.006) (end 120.724 101.006) (width 0.2) (layer "F.Cu") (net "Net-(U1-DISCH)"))
 (segment (start 114.175 97.825) (end 117.356 101.006) (width 0.2) (layer "F.Cu") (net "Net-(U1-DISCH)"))
 (segment (start 114.175 95.5) (end 114.175 97.825) (width 0.2) (layer "F.Cu") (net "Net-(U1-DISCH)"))
 (segment (start 125.15 105.5) (end 123.2 105.5) (width 0.2) (layer "F.Cu") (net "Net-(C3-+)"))
 (segment (start 123.2 105.5) (end 123.1 105.4) (width 0.2) (layer "F.Cu") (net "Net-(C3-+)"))
 (segment (start 132.5 114.5) (end 132.5 114.55) (width 0.2) (layer "F.Cu") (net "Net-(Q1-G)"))
 (segment (start 116 103.5) (end 115.5 103) (width 0.2) (layer "F.Cu") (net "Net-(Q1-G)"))
 (segment (start 116.15 103.85) (end 116 104) (width 0.2) (layer "F.Cu") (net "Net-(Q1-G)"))
 (segment (start 130.5 112.5) (end 132.5 114.5) (width 0.2) (layer "F.Cu") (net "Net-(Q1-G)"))
 (segment (start 116.15 102.5) (end 116.15 103.85) (width 0.2) (layer "F.Cu") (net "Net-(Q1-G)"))
 (via (at 115.5 103) (size 0.6) (drill 0.3) (layers "F.Cu" "B.Cu") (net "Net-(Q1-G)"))
 (via (at 130.5 112.5) (size 0.6) (drill 0.3) (layers "F.Cu" "B.Cu") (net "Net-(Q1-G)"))
 (segment (start 130.5 108.5) (end 130.5 112.5) (width 0.2) (layer "B.Cu") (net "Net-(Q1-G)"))
 (segment (start 115.5 103) (end 113.5 105) (width 0.2) (layer "B.Cu") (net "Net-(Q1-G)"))
 (segment (start 113.5 105) (end 113.5 109) (width 0.2) (layer "B.Cu") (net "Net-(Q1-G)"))
 (segment (start 113.5 109) (end 130 109) (width 0.2) (layer "B.Cu") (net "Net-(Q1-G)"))
 (segment (start 130 109) (end 130.5 108.5) (width 0.2) (layer "B.Cu") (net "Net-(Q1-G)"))
 (segment (start 114.7 104) (end 115.4 104.7) (width 0.2) (layer "F.Cu") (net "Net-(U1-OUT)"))
 (segment (start 115.4 104.7) (end 115.4 106.3) (width 0.2) (layer "F.Cu") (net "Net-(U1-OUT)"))
 (segment (start 115.4 106.3) (end 118.446043 106.3) (width 0.2) (layer "F.Cu") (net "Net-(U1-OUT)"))
 (segment (start 118.446043 106.3) (end 119.1 105.646043) (width 0.2) (layer "F.Cu") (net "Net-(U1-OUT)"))
 (segment (start 119.1 105.646043) (end 119.1 104.6) (width 0.2) (layer "F.Cu") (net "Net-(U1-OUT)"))
 (segment (start 119.1 104.6) (end 118.63 104.13) (width 0.2) (layer "F.Cu") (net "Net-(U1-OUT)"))
 (segment (start 118.63 104.13) (end 117.9 104.13) (width 0.2) (layer "F.Cu") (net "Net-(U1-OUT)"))
 (segment (start 114.35 104) (end 114.7 104) (width 0.2) (layer "F.Cu") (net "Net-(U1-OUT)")))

